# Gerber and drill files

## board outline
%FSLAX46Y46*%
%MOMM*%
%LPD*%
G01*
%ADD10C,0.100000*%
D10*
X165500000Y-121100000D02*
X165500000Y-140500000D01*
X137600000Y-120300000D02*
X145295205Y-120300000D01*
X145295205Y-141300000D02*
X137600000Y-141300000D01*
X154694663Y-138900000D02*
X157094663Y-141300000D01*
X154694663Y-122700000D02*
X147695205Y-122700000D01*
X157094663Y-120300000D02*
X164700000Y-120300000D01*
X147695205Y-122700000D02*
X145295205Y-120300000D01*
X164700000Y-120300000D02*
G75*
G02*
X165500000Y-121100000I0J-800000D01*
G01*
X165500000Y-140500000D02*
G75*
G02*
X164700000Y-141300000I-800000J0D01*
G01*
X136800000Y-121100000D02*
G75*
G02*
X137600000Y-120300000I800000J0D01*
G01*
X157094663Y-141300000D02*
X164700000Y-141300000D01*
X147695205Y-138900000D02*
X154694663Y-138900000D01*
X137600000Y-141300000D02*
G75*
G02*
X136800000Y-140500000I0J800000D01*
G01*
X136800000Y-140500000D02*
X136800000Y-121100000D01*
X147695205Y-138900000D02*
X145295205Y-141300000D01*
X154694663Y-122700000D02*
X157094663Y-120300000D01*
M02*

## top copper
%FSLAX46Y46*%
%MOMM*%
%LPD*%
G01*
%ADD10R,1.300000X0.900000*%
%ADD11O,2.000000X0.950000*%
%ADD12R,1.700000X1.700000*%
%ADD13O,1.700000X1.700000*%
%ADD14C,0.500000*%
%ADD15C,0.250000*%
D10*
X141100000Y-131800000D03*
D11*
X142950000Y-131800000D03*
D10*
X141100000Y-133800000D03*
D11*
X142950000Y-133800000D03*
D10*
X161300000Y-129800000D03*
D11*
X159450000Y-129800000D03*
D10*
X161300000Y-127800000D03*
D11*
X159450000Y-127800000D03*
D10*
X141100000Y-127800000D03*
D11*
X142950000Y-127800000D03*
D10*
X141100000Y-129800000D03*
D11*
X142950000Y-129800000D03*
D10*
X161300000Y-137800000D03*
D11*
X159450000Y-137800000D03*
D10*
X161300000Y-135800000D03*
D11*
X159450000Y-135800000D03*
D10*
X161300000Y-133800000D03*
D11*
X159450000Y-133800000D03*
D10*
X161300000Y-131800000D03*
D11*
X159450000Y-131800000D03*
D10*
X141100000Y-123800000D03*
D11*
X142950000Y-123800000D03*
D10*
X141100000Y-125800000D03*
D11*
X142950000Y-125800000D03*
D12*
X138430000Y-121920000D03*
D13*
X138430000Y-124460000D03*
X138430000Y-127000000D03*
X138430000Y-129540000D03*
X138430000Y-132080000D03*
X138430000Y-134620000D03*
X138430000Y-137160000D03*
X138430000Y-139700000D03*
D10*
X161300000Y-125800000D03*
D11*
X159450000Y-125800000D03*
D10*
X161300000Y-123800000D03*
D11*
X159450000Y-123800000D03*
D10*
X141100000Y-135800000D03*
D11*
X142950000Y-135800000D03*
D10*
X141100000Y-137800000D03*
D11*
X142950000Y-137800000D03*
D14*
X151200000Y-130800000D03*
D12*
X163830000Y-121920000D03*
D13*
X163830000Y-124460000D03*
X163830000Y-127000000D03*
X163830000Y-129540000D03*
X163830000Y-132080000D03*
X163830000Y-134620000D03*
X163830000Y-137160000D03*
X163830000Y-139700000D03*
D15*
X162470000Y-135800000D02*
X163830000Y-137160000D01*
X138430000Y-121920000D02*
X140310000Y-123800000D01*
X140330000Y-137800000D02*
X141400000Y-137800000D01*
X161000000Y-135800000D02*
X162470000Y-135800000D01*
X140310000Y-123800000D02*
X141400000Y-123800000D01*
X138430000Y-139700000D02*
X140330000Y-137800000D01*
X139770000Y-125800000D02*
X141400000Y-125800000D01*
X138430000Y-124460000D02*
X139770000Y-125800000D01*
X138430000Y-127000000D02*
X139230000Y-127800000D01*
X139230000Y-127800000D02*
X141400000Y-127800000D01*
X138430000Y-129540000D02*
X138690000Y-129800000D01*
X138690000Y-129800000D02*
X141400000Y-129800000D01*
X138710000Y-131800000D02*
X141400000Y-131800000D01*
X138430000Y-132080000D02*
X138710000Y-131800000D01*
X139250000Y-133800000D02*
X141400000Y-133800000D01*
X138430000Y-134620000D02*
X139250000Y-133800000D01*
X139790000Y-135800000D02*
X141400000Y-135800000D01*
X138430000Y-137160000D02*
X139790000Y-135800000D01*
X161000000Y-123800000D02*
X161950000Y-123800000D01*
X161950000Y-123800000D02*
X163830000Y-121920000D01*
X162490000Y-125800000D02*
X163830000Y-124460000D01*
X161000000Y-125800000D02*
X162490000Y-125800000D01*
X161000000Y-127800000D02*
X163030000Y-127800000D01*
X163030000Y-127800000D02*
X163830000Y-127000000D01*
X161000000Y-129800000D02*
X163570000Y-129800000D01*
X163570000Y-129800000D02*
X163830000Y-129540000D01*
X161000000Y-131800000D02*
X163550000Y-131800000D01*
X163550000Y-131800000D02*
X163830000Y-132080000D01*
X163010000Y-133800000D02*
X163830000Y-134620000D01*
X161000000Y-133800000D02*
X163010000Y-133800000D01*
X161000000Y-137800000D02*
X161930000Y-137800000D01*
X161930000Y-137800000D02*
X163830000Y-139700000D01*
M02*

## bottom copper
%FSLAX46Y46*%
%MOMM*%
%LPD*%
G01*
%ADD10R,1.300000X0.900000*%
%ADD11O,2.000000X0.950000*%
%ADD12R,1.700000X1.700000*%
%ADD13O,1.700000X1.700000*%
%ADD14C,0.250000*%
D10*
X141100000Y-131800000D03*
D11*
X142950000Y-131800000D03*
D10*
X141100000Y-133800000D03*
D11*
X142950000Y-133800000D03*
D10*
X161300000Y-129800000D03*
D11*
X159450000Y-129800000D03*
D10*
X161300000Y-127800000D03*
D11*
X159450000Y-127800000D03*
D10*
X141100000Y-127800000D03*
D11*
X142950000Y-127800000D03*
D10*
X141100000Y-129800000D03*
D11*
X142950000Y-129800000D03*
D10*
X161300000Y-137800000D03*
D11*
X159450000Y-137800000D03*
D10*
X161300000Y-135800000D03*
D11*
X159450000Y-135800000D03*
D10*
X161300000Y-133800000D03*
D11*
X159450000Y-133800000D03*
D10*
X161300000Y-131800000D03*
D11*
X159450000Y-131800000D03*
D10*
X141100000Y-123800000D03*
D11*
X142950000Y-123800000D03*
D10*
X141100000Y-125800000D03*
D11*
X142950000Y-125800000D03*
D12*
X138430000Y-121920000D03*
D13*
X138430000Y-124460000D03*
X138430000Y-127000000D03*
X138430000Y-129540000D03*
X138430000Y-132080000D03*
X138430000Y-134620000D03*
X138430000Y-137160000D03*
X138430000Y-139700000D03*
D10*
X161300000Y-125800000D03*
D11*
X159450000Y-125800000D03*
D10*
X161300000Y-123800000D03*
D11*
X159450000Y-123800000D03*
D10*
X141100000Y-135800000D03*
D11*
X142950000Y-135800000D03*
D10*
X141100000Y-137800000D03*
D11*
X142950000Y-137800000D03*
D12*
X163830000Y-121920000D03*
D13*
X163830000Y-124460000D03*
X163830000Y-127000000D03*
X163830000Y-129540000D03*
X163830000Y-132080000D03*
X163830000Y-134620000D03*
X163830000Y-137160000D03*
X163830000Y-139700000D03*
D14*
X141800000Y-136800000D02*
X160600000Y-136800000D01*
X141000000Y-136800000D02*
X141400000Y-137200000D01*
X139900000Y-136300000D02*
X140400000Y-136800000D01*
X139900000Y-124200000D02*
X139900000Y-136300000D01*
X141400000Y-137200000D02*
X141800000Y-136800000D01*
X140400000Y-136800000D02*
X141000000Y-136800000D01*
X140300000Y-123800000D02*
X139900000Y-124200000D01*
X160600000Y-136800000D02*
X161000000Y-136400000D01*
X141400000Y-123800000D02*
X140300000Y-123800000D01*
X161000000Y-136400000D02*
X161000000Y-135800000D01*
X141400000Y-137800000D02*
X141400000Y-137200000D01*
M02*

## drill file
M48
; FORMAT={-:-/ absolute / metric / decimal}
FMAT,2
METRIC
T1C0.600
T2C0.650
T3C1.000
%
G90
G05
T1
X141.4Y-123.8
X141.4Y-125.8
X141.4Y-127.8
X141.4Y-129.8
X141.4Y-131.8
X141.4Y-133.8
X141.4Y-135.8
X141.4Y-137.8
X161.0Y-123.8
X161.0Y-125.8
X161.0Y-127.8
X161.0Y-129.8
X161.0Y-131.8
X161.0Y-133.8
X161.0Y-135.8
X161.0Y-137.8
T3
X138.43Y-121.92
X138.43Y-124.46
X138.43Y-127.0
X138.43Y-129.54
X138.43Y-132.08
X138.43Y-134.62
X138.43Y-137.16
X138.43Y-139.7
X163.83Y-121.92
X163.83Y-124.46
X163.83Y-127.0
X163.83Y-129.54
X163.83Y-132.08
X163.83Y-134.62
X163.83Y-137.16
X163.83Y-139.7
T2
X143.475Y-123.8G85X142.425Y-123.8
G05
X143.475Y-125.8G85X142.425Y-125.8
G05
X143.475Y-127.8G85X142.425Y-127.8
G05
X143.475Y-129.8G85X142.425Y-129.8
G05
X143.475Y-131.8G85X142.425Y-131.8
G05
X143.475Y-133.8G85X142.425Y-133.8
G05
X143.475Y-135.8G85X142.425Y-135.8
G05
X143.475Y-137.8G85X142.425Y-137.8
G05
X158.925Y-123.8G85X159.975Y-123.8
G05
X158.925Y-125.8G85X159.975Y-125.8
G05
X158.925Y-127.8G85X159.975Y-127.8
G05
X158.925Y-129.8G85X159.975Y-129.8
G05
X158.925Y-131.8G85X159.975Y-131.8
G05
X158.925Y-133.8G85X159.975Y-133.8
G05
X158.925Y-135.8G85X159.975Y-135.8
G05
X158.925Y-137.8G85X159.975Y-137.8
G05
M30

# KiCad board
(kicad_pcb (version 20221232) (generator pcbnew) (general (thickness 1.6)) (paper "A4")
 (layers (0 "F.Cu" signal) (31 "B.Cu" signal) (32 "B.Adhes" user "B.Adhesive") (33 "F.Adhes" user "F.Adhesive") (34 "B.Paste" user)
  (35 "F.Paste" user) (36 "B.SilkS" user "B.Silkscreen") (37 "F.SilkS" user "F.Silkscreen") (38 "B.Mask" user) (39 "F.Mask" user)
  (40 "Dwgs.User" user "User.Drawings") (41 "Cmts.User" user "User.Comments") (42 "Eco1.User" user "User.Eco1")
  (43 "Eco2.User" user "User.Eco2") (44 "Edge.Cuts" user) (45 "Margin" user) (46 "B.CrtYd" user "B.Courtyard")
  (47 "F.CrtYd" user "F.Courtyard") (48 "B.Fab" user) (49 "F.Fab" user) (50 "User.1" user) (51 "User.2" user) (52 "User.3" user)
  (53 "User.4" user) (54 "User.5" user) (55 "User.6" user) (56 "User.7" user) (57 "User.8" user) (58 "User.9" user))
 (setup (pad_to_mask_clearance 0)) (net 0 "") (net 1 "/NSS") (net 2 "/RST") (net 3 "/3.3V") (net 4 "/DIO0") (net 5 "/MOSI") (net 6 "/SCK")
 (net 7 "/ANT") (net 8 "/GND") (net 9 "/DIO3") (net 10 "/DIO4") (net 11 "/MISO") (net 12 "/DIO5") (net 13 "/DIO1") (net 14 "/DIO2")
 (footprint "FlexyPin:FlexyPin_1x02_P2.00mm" (layer "F.Cu") (at 141.4 131.8)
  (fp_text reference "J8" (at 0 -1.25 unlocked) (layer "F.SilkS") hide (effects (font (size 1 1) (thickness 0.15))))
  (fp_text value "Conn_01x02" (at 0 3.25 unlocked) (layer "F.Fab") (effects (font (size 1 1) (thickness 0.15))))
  (pad "1" thru_hole rect (at 0 0) (size 1.3 0.9) (drill 0.6 (offset -0.3 0)) (layers *.Cu *.Mask) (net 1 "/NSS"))
  (pad "1" thru_hole oval (at 1.55 0 180) (size 2 0.95) (drill oval 1.7 0.65) (layers *.Cu *.Mask) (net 1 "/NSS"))
  (pad "2" thru_hole rect (at 0 2) (size 1.3 0.9) (drill 0.6 (offset -0.3 0)) (layers *.Cu *.Mask) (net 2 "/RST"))
  (pad "2" thru_hole oval (at 1.55 2 180) (size 2 0.95) (drill oval 1.7 0.65) (layers *.Cu *.Mask) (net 2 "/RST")))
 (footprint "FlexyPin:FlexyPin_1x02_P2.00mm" (layer "F.Cu") (at 161 129.8 180)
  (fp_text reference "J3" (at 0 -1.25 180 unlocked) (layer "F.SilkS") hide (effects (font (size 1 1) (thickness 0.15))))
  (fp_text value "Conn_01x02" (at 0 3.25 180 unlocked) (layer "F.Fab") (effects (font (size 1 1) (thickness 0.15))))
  (pad "1" thru_hole rect (at 0 0 180) (size 1.3 0.9) (drill 0.6 (offset -0.3 0)) (layers *.Cu *.Mask) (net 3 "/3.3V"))
  (pad "1" thru_hole oval (at 1.55 0) (size 2 0.95) (drill oval 1.7 0.65) (layers *.Cu *.Mask) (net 3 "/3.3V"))
  (pad "2" thru_hole rect (at 0 2 180) (size 1.3 0.9) (drill 0.6 (offset -0.3 0)) (layers *.Cu *.Mask) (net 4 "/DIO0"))
  (pad "2" thru_hole oval (at 1.55 2) (size 2 0.95) (drill oval 1.7 0.65) (layers *.Cu *.Mask) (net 4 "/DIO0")))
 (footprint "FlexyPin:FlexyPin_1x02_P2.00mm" (layer "F.Cu") (at 141.4 127.8)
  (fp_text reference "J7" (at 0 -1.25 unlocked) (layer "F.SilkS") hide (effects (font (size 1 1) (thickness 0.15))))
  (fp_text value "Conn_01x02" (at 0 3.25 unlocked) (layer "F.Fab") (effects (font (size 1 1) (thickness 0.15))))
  (pad "1" thru_hole rect (at 0 0) (size 1.3 0.9) (drill 0.6 (offset -0.3 0)) (layers *.Cu *.Mask) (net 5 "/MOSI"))
  (pad "1" thru_hole oval (at 1.55 0 180) (size 2 0.95) (drill oval 1.7 0.65) (layers *.Cu *.Mask) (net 5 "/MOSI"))
  (pad "2" thru_hole rect (at 0 2) (size 1.3 0.9) (drill 0.6 (offset -0.3 0)) (layers *.Cu *.Mask) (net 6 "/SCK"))
  (pad "2" thru_hole oval (at 1.55 2 180) (size 2 0.95) (drill oval 1.7 0.65) (layers *.Cu *.Mask) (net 6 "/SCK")))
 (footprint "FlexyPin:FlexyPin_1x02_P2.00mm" (layer "F.Cu") (at 161 137.8 180)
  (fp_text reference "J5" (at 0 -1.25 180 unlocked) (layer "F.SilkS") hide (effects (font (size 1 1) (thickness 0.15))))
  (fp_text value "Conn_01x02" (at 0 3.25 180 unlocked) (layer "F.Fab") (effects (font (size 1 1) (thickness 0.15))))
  (pad "1" thru_hole rect (at 0 0 180) (size 1.3 0.9) (drill 0.6 (offset -0.3 0)) (layers *.Cu *.Mask) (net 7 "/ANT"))
  (pad "1" thru_hole oval (at 1.55 0) (size 2 0.95) (drill oval 1.7 0.65) (layers *.Cu *.Mask) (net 7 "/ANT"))
  (pad "2" thru_hole rect (at 0 2 180) (size 1.3 0.9) (drill 0.6 (offset -0.3 0)) (layers *.Cu *.Mask) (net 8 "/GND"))
  (pad "2" thru_hole oval (at 1.55 2) (size 2 0.95) (drill oval 1.7 0.65) (layers *.Cu *.Mask) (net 8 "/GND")))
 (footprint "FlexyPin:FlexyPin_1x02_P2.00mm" (layer "F.Cu") (at 161 133.8 180)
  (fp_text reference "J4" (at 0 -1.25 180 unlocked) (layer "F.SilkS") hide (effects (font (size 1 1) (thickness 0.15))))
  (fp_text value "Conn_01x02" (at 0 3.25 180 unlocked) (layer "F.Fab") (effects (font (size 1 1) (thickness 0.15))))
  (pad "1" thru_hole rect (at 0 0 180) (size 1.3 0.9) (drill 0.6 (offset -0.3 0)) (layers *.Cu *.Mask) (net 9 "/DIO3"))
  (pad "1" thru_hole oval (at 1.55 0) (size 2 0.95) (drill oval 1.7 0.65) (layers *.Cu *.Mask) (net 9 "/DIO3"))
  (pad "2" thru_hole rect (at 0 2 180) (size 1.3 0.9) (drill 0.6 (offset -0.3 0)) (layers *.Cu *.Mask) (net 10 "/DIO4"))
  (pad "2" thru_hole oval (at 1.55 2) (size 2 0.95) (drill oval 1.7 0.65) (layers *.Cu *.Mask) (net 10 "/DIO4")))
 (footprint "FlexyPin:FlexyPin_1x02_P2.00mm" (layer "F.Cu") (at 141.4 123.8)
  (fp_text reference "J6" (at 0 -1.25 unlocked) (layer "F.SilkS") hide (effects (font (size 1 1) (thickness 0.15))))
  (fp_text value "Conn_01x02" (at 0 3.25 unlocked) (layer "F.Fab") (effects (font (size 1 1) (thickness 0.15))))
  (pad "1" thru_hole rect (at 0 0) (size 1.3 0.9) (drill 0.6 (offset -0.3 0)) (layers *.Cu *.Mask) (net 8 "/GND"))
  (pad "1" thru_hole oval (at 1.55 0 180) (size 2 0.95) (drill oval 1.7 0.65) (layers *.Cu *.Mask) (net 8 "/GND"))
  (pad "2" thru_hole rect (at 0 2) (size 1.3 0.9) (drill 0.6 (offset -0.3 0)) (layers *.Cu *.Mask) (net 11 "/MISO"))
  (pad "2" thru_hole oval (at 1.55 2 180) (size 2 0.95) (drill oval 1.7 0.65) (layers *.Cu *.Mask) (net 11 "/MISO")))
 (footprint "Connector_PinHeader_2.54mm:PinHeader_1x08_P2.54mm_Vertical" (layer "F.Cu") (at 138.43 121.92)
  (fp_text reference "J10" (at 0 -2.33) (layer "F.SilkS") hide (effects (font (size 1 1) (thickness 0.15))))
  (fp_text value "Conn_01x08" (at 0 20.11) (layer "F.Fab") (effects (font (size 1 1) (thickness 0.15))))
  (pad "1" thru_hole rect locked (at 0 0) (size 1.7 1.7) (drill 1) (layers *.Cu *.Mask) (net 8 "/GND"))
  (pad "2" thru_hole oval locked (at 0 2.54) (size 1.7 1.7) (drill 1) (layers *.Cu *.Mask) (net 11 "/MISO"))
  (pad "3" thru_hole oval locked (at 0 5.08) (size 1.7 1.7) (drill 1) (layers *.Cu *.Mask) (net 5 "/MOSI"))
  (pad "4" thru_hole oval locked (at 0 7.62) (size 1.7 1.7) (drill 1) (layers *.Cu *.Mask) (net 6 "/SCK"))
  (pad "5" thru_hole oval locked (at 0 10.16) (size 1.7 1.7) (drill 1) (layers *.Cu *.Mask) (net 1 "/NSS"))
  (pad "6" thru_hole oval locked (at 0 12.7) (size 1.7 1.7) (drill 1) (layers *.Cu *.Mask) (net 2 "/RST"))
  (pad "7" thru_hole oval locked (at 0 15.24) (size 1.7 1.7) (drill 1) (layers *.Cu *.Mask) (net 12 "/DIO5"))
  (pad "8" thru_hole oval locked (at 0 17.78) (size 1.7 1.7) (drill 1) (layers *.Cu *.Mask) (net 8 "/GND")))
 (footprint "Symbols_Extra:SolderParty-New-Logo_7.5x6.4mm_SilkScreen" (layer "F.Cu") (at 151.2 135.5)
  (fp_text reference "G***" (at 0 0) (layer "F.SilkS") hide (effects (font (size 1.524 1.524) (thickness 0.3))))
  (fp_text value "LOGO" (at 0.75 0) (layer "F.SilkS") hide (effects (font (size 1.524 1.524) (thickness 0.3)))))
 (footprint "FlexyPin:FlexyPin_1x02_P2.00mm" (layer "F.Cu") (at 161 125.8 180)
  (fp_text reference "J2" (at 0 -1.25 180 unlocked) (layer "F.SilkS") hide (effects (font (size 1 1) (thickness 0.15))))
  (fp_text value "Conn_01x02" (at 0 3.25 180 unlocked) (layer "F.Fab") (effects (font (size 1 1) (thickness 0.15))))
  (pad "1" thru_hole rect (at 0 0 180) (size 1.3 0.9) (drill 0.6 (offset -0.3 0)) (layers *.Cu *.Mask) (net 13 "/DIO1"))
  (pad "1" thru_hole oval (at 1.55 0) (size 2 0.95) (drill oval 1.7 0.65) (layers *.Cu *.Mask) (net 13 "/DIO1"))
  (pad "2" thru_hole rect (at 0 2 180) (size 1.3 0.9) (drill 0.6 (offset -0.3 0)) (layers *.Cu *.Mask) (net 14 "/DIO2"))
  (pad "2" thru_hole oval (at 1.55 2) (size 2 0.95) (drill oval 1.7 0.65) (layers *.Cu *.Mask) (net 14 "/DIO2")))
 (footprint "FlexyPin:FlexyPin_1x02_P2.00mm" (layer "F.Cu") (at 141.4 135.8)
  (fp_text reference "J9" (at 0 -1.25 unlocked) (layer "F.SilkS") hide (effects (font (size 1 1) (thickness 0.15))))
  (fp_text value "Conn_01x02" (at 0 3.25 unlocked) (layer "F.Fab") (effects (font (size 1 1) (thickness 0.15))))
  (pad "1" thru_hole rect (at 0 0) (size 1.3 0.9) (drill 0.6 (offset -0.3 0)) (layers *.Cu *.Mask) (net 12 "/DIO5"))
  (pad "1" thru_hole oval (at 1.55 0 180) (size 2 0.95) (drill oval 1.7 0.65) (layers *.Cu *.Mask) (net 12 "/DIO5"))
  (pad "2" thru_hole rect (at 0 2) (size 1.3 0.9) (drill 0.6 (offset -0.3 0)) (layers *.Cu *.Mask) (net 8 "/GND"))
  (pad "2" thru_hole oval (at 1.55 2 180) (size 2 0.95) (drill oval 1.7 0.65) (layers *.Cu *.Mask) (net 8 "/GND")))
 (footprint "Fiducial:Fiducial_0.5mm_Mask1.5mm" (layer "F.Cu") (at 151.2 130.8)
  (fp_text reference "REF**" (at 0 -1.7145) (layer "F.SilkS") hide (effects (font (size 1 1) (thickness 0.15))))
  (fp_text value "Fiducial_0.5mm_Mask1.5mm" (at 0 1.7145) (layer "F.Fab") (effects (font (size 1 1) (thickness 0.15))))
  (pad "" smd circle (at 0 0) (size 0.5 0.5) (layers "F.Cu") (solder_mask_margin 0.5) (clearance 0.5)))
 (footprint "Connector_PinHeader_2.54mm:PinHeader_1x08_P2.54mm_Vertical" (layer "F.Cu") (at 163.83 121.92)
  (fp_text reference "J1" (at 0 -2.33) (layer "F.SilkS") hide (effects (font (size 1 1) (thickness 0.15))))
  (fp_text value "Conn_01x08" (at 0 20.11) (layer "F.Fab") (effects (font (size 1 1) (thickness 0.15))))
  (pad "1" thru_hole rect locked (at 0 0) (size 1.7 1.7) (drill 1) (layers *.Cu *.Mask) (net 14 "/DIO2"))
  (pad "2" thru_hole oval locked (at 0 2.54) (size 1.7 1.7) (drill 1) (layers *.Cu *.Mask) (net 13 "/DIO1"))
  (pad "3" thru_hole oval locked (at 0 5.08) (size 1.7 1.7) (drill 1) (layers *.Cu *.Mask) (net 4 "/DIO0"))
  (pad "4" thru_hole oval locked (at 0 7.62) (size 1.7 1.7) (drill 1) (layers *.Cu *.Mask) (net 3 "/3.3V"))
  (pad "5" thru_hole oval locked (at 0 10.16) (size 1.7 1.7) (drill 1) (layers *.Cu *.Mask) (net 10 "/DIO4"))
  (pad "6" thru_hole oval locked (at 0 12.7) (size 1.7 1.7) (drill 1) (layers *.Cu *.Mask) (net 9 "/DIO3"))
  (pad "7" thru_hole oval locked (at 0 15.24) (size 1.7 1.7) (drill 1) (layers *.Cu *.Mask) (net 8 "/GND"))
  (pad "8" thru_hole oval locked (at 0 17.78) (size 1.7 1.7) (drill 1) (layers *.Cu *.Mask) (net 7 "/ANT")))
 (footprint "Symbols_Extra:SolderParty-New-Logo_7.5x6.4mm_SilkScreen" (layer "B.Cu") (at 150.719476 135 180)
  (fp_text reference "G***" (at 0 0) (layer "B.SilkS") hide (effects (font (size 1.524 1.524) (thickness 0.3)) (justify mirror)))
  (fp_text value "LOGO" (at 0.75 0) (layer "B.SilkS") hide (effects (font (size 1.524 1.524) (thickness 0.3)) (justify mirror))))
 (gr_line (start 165.5 121.1) (end 165.5 140.5) (stroke (width 0.1) (type solid)) (layer "Edge.Cuts"))
 (gr_line (start 137.6 120.3) (end 145.295205 120.3) (stroke (width 0.1) (type solid)) (layer "Edge.Cuts"))
 (gr_line (start 145.295205 141.3) (end 137.6 141.3) (stroke (width 0.1) (type solid)) (layer "Edge.Cuts"))
 (gr_line (start 154.694663 138.9) (end 157.094663 141.3) (stroke (width 0.1) (type solid)) (layer "Edge.Cuts"))
 (gr_line (start 154.694663 122.7) (end 147.695205 122.7) (stroke (width 0.1) (type solid)) (layer "Edge.Cuts"))
 (gr_line (start 157.094663 120.3) (end 164.7 120.3) (stroke (width 0.1) (type solid)) (layer "Edge.Cuts"))
 (gr_line (start 147.695205 122.7) (end 145.295205 120.3) (stroke (width 0.1) (type solid)) (layer "Edge.Cuts"))
 (gr_arc (start 164.7 120.3) (mid 165.265685 120.534315) (end 165.5 121.1) (stroke (width 0.1) (type solid)) (layer "Edge.Cuts"))
 (gr_arc (start 165.5 140.5) (mid 165.265685 141.065685) (end 164.7 141.3) (stroke (width 0.1) (type solid)) (layer "Edge.Cuts"))
 (gr_arc (start 136.8 121.1) (mid 137.034315 120.534315) (end 137.6 120.3) (stroke (width 0.1) (type solid)) (layer "Edge.Cuts"))
 (gr_line (start 157.094663 141.3) (end 164.7 141.3) (stroke (width 0.1) (type solid)) (layer "Edge.Cuts"))
 (gr_line (start 147.695205 138.9) (end 154.694663 138.9) (stroke (width 0.1) (type solid)) (layer "Edge.Cuts"))
 (gr_arc (start 137.6 141.3) (mid 137.034315 141.065685) (end 136.8 140.5) (stroke (width 0.1) (type solid)) (layer "Edge.Cuts"))
 (gr_line (start 136.8 140.5) (end 136.8 121.1) (stroke (width 0.1) (type solid)) (layer "Edge.Cuts"))
 (gr_line (start 147.695205 138.9) (end 145.295205 141.3) (stroke (width 0.1) (type solid)) (layer "Edge.Cuts"))
 (gr_line (start 154.694663 122.7) (end 157.094663 120.3) (stroke (width 0.1) (type solid)) (layer "Edge.Cuts"))
 (segment (start 162.47 135.8) (end 163.83 137.16) (width 0.25) (layer "F.Cu") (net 8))
 (segment (start 138.43 121.92) (end 140.31 123.8) (width 0.25) (layer "F.Cu") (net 8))
 (segment (start 140.33 137.8) (end 141.4 137.8) (width 0.25) (layer "F.Cu") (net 8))
 (segment (start 161 135.8) (end 162.47 135.8) (width 0.25) (layer "F.Cu") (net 8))
 (segment (start 140.31 123.8) (end 141.4 123.8) (width 0.25) (layer "F.Cu") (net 8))
 (segment (start 138.43 139.7) (end 140.33 137.8) (width 0.25) (layer "F.Cu") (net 8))
 (segment (start 141.8 136.8) (end 160.6 136.8) (width 0.25) (layer "B.Cu") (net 8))
 (segment (start 141 136.8) (end 141.4 137.2) (width 0.25) (layer "B.Cu") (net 8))
 (segment (start 139.9 136.3) (end 140.4 136.8) (width 0.25) (layer "B.Cu") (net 8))
 (segment (start 139.9 124.2) (end 139.9 136.3) (width 0.25) (layer "B.Cu") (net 8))
 (segment (start 141.4 137.2) (end 141.8 136.8) (width 0.25) (layer "B.Cu") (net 8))
 (segment (start 140.4 136.8) (end 141 136.8) (width 0.25) (layer "B.Cu") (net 8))
 (segment (start 140.3 123.8) (end 139.9 124.2) (width 0.25) (layer "B.Cu") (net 8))
 (segment (start 160.6 136.8) (end 161 136.4) (width 0.25) (layer "B.Cu") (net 8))
 (segment (start 141.4 123.8) (end 140.3 123.8) (width 0.25) (layer "B.Cu") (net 8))
 (segment (start 161 136.4) (end 161 135.8) (width 0.25) (layer "B.Cu") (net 8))
 (segment (start 141.4 137.8) (end 141.4 137.2) (width 0.25) (layer "B.Cu") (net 8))
 (segment (start 139.77 125.8) (end 141.4 125.8) (width 0.25) (layer "F.Cu") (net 11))
 (segment (start 138.43 124.46) (end 139.77 125.8) (width 0.25) (layer "F.Cu") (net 11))
 (segment (start 138.43 127) (end 139.23 127.8) (width 0.25) (layer "F.Cu") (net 5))
 (segment (start 139.23 127.8) (end 141.4 127.8) (width 0.25) (layer "F.Cu") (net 5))
 (segment (start 138.43 129.54) (end 138.69 129.8) (width 0.25) (layer "F.Cu") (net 6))
 (segment (start 138.69 129.8) (end 141.4 129.8) (width 0.25) (layer "F.Cu") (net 6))
 (segment (start 138.71 131.8) (end 141.4 131.8) (width 0.25) (layer "F.Cu") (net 1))
 (segment (start 138.43 132.08) (end 138.71 131.8) (width 0.25) (layer "F.Cu") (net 1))
 (segment (start 139.25 133.8) (end 141.4 133.8) (width 0.25) (layer "F.Cu") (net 2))
 (segment (start 138.43 134.62) (end 139.25 133.8) (width 0.25) (layer "F.Cu") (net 2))
 (segment (start 139.79 135.8) (end 141.4 135.8) (width 0.25) (layer "F.Cu") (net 12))
 (segment (start 138.43 137.16) (end 139.79 135.8) (width 0.25) (layer "F.Cu") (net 12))
 (segment (start 161 123.8) (end 161.95 123.8) (width 0.25) (layer "F.Cu") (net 14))
 (segment (start 161.95 123.8) (end 163.83 121.92) (width 0.25) (layer "F.Cu") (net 14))
 (segment (start 162.49 125.8) (end 163.83 124.46) (width 0.25) (layer "F.Cu") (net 13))
 (segment (start 161 125.8) (end 162.49 125.8) (width 0.25) (layer "F.Cu") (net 13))
 (segment (start 161 127.8) (end 163.03 127.8) (width 0.25) (layer "F.Cu") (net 4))
 (segment (start 163.03 127.8) (end 163.83 127) (width 0.25) (layer "F.Cu") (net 4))
 (segment (start 161 129.8) (end 163.57 129.8) (width 0.25) (layer "F.Cu") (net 3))
 (segment (start 163.57 129.8) (end 163.83 129.54) (width 0.25) (layer "F.Cu") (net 3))
 (segment (start 161 131.8) (end 163.55 131.8) (width 0.25) (layer "F.Cu") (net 10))
 (segment (start 163.55 131.8) (end 163.83 132.08) (width 0.25) (layer "F.Cu") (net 10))
 (segment (start 163.01 133.8) (end 163.83 134.62) (width 0.25) (layer "F.Cu") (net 9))
 (segment (start 161 133.8) (end 163.01 133.8) (width 0.25) (layer "F.Cu") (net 9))
 (segment (start 161 137.8) (end 161.93 137.8) (width 0.25) (layer "F.Cu") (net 7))
 (segment (start 161.93 137.8) (end 163.83 139.7) (width 0.25) (layer "F.Cu") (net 7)))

